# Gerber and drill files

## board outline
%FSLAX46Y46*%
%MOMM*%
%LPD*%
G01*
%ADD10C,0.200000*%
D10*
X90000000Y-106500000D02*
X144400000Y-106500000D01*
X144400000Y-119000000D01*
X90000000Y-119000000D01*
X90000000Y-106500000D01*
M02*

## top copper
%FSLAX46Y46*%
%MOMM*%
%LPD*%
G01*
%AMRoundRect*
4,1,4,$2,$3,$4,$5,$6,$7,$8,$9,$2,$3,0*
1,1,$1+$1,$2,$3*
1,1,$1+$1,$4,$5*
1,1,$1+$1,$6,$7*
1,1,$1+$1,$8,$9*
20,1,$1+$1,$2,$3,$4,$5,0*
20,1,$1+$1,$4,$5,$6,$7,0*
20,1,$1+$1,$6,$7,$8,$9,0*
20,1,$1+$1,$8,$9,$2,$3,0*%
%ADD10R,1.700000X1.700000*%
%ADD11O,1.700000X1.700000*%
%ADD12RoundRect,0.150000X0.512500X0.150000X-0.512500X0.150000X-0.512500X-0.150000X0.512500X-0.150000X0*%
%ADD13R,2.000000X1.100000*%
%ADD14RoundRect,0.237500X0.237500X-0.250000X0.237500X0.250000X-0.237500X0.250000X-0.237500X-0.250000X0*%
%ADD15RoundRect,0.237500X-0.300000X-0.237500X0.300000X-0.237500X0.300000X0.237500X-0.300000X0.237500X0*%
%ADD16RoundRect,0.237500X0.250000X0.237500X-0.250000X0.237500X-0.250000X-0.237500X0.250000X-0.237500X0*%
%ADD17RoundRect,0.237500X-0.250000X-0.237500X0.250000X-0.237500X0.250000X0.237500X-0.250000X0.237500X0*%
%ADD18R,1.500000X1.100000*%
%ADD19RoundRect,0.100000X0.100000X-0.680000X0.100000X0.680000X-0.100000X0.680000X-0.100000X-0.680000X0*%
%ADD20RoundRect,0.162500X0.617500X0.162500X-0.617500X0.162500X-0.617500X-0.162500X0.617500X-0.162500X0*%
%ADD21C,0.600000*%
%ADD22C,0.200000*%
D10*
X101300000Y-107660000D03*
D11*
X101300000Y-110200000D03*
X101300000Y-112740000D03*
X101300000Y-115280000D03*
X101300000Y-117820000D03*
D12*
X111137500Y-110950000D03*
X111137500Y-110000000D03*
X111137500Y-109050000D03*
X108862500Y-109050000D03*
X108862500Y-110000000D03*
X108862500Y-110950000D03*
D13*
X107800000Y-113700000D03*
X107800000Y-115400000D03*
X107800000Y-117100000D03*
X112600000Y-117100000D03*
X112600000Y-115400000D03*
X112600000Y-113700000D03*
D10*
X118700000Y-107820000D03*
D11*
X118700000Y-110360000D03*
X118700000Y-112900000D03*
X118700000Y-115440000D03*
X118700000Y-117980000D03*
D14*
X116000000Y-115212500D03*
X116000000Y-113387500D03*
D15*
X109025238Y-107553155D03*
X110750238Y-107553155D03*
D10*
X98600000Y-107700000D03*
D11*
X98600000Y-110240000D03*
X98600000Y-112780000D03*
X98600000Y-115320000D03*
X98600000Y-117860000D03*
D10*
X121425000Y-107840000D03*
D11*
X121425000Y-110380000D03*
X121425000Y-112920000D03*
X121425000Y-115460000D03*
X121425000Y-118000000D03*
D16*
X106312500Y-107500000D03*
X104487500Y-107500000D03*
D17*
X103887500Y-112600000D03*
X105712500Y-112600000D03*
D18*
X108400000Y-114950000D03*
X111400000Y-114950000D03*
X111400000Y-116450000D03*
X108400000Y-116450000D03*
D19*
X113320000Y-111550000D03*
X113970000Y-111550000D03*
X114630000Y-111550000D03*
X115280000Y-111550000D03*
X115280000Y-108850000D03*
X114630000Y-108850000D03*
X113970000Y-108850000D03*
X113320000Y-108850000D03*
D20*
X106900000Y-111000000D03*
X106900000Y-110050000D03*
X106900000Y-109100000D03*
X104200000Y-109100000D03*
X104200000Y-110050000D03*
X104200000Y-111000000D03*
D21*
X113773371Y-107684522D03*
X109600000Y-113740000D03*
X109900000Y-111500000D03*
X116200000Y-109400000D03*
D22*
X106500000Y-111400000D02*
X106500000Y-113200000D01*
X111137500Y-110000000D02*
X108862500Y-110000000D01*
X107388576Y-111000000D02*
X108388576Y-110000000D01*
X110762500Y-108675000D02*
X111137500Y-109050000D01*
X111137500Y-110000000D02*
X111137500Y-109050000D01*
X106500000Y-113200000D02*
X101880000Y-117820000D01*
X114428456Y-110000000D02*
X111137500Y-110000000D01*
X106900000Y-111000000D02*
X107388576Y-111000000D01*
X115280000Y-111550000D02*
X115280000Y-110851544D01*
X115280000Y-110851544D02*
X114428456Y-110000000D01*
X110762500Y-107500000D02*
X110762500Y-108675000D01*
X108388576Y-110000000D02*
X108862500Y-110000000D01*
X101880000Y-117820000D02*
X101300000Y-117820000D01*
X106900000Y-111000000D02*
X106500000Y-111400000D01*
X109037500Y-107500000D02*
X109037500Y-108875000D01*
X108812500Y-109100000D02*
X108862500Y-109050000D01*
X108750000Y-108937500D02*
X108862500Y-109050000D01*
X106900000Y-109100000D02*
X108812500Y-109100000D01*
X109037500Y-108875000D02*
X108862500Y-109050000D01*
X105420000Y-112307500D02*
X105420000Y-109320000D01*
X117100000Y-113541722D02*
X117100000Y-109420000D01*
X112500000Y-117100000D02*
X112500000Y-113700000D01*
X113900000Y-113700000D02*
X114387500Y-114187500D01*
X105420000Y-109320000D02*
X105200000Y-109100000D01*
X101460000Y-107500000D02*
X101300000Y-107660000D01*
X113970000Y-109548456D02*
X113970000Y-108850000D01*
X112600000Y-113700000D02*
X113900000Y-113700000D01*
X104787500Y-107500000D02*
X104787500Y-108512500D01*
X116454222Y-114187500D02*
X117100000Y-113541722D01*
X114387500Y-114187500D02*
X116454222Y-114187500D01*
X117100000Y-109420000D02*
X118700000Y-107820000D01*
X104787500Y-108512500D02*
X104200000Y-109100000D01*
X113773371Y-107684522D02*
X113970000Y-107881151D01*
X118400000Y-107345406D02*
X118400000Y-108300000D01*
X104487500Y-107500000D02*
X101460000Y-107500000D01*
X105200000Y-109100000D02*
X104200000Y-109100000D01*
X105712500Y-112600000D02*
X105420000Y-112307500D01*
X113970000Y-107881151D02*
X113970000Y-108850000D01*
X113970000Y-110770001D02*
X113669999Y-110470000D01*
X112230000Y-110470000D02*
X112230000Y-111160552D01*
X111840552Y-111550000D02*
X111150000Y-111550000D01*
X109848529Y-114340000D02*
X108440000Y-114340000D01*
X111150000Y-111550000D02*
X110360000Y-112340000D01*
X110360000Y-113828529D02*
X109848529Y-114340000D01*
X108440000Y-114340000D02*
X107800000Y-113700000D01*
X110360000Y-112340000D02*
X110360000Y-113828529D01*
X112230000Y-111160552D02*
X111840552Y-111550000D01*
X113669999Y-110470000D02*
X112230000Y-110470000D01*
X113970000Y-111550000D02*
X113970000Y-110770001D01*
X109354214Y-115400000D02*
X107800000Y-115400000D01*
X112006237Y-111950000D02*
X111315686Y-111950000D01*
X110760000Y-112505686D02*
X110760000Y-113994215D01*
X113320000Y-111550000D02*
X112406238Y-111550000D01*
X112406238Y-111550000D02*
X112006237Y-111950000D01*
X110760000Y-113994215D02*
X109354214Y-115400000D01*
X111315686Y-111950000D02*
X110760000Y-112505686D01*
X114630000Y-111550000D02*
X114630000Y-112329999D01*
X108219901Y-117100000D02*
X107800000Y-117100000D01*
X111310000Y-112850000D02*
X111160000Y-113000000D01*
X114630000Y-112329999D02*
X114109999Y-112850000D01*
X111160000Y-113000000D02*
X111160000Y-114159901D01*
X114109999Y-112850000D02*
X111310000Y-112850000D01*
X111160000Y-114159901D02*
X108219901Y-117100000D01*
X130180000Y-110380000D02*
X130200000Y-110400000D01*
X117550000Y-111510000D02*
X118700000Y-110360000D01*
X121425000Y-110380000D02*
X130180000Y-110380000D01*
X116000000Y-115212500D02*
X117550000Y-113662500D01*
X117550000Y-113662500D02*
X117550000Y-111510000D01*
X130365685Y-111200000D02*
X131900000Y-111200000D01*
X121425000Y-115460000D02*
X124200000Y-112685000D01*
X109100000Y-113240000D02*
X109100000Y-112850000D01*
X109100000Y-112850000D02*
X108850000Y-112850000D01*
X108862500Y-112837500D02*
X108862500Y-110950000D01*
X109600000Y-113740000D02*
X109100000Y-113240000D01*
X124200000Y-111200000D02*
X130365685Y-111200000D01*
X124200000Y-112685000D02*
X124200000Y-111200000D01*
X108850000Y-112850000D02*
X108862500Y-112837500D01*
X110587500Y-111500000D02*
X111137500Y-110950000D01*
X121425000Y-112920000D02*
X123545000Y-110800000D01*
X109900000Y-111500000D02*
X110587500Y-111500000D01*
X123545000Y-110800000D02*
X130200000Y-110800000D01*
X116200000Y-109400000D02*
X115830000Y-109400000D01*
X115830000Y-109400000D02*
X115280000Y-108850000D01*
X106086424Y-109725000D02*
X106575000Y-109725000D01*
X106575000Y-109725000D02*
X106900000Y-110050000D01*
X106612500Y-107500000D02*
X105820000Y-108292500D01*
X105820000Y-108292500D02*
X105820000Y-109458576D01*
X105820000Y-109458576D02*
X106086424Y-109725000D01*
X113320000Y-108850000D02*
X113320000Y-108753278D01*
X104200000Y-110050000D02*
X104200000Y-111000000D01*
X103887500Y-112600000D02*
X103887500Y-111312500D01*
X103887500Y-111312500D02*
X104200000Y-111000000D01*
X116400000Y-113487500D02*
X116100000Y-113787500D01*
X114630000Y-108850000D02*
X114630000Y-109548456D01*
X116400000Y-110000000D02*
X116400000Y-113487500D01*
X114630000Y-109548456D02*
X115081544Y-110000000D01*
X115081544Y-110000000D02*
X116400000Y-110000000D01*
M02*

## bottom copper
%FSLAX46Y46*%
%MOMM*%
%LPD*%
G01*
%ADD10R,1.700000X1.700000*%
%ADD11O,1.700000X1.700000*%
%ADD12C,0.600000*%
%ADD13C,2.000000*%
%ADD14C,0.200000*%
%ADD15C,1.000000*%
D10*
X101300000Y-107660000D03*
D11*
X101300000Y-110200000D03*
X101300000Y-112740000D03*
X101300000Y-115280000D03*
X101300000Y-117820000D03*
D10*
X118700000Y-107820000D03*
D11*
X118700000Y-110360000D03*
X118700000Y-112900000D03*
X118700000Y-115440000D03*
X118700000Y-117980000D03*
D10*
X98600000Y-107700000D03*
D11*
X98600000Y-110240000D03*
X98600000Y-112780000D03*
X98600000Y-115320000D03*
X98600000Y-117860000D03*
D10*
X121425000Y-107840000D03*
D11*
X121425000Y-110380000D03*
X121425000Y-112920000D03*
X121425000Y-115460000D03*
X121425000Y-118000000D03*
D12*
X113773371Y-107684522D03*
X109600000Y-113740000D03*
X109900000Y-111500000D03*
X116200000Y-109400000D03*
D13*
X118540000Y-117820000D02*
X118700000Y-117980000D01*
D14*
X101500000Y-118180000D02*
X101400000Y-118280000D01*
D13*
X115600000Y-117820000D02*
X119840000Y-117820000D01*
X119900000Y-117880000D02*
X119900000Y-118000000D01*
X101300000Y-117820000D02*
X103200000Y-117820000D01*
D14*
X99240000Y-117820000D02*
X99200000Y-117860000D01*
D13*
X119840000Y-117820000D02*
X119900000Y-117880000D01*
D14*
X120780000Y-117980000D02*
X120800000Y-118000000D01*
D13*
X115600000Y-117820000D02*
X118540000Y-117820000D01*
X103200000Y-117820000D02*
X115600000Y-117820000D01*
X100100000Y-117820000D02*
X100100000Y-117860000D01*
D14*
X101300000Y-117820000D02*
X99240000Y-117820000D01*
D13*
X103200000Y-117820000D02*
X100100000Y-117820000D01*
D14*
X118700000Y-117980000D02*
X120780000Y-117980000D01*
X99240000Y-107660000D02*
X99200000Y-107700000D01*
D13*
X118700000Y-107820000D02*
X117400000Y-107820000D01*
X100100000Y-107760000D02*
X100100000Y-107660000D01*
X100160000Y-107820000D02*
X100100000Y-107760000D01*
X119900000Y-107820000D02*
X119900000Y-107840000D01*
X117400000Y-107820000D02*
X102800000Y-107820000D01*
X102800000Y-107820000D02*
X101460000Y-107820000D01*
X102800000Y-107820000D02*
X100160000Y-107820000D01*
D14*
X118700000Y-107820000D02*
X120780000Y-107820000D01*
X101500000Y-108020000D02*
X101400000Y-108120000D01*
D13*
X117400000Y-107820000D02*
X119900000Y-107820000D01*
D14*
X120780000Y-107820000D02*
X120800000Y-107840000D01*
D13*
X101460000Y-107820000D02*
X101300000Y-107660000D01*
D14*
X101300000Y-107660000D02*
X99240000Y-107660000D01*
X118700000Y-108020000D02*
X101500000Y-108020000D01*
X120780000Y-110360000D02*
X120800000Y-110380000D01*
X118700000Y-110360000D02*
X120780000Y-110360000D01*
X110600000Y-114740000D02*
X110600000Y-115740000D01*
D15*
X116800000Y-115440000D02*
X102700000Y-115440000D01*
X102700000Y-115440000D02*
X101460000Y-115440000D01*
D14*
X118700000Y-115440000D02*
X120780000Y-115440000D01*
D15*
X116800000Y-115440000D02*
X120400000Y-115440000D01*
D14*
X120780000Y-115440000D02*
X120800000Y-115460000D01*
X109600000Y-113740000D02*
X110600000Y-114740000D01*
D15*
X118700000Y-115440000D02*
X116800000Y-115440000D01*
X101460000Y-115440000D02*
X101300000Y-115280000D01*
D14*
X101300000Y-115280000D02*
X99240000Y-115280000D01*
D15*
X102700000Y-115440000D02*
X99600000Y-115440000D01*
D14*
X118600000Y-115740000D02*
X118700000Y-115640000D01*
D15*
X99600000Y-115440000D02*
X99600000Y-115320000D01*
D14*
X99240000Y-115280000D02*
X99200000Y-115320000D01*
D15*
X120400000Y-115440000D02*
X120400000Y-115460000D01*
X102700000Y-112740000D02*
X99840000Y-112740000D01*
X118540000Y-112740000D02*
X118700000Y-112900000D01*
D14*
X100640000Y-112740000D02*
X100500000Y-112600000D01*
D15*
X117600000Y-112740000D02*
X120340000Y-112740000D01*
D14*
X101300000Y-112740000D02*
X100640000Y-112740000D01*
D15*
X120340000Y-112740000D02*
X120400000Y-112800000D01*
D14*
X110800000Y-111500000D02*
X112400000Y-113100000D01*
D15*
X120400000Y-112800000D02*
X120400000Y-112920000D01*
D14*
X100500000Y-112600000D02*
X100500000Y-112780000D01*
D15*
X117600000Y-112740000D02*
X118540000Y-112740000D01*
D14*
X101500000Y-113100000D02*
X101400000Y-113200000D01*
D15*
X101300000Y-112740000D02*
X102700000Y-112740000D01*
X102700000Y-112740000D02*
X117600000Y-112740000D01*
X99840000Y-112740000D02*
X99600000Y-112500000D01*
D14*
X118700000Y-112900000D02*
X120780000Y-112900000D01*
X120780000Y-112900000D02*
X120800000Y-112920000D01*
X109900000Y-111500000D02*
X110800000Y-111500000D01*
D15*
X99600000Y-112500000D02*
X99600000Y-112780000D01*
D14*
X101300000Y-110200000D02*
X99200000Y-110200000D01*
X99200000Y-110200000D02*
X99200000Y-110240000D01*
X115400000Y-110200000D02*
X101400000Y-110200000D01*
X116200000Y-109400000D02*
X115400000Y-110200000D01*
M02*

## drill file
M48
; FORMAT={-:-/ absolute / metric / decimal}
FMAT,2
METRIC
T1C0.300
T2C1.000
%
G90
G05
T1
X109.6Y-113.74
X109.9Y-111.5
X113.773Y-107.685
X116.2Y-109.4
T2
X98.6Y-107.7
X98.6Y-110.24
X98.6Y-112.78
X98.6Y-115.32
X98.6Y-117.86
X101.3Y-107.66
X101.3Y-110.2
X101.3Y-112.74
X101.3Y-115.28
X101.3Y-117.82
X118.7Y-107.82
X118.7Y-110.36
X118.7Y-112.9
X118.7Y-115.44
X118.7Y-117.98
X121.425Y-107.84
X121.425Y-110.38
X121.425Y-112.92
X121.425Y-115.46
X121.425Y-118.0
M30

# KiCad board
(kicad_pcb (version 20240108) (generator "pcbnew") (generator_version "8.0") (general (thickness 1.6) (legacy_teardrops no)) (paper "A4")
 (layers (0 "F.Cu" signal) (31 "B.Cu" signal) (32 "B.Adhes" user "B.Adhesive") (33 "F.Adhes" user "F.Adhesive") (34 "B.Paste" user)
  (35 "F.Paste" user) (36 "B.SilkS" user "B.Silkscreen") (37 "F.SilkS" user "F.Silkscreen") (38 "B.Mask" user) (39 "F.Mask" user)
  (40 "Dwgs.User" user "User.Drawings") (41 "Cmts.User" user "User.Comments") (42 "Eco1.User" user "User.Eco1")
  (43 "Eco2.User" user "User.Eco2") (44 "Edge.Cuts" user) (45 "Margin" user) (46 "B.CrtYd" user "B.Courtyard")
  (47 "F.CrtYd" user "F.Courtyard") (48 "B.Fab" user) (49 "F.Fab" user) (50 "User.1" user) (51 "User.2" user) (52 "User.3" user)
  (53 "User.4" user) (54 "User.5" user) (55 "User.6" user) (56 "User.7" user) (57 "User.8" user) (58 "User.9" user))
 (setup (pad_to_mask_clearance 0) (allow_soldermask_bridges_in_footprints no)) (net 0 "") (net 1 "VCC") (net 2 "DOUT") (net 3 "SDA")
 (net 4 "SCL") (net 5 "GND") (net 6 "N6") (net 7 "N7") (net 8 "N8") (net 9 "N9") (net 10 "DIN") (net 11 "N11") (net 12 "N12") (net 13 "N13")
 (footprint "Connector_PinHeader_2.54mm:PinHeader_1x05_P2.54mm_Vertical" (layer "F.Cu") (at 101.3 107.66)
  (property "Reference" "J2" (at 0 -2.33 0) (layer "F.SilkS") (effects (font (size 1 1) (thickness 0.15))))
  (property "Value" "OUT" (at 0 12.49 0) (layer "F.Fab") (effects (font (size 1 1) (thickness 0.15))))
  (pad "1" thru_hole rect (at 0 0) (size 1.7 1.7) (drill 1) (layers "*.Cu" "*.Mask") (remove_unused_layers no) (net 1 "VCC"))
  (pad "2" thru_hole oval (at 0 2.54) (size 1.7 1.7) (drill 1) (layers "*.Cu" "*.Mask") (remove_unused_layers no) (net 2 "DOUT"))
  (pad "3" thru_hole oval (at 0 5.08) (size 1.7 1.7) (drill 1) (layers "*.Cu" "*.Mask") (remove_unused_layers no) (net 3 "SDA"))
  (pad "4" thru_hole oval (at 0 7.62) (size 1.7 1.7) (drill 1) (layers "*.Cu" "*.Mask") (remove_unused_layers no) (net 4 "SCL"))
  (pad "5" thru_hole oval (at 0 10.16) (size 1.7 1.7) (drill 1) (layers "*.Cu" "*.Mask") (remove_unused_layers no) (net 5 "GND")))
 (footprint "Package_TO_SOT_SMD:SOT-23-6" (layer "F.Cu") (at 110 110 180)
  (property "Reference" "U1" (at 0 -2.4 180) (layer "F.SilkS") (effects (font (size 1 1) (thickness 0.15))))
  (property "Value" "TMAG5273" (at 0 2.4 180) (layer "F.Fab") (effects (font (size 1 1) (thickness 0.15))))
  (pad "1" smd roundrect (at -1.1375 -0.95 180) (size 1.325 0.6) (layers "F.Cu" "F.Paste" "F.Mask") (roundrect_rratio 0.25) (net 3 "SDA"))
  (pad "2" smd roundrect (at -1.1375 0 180) (size 1.325 0.6) (layers "F.Cu" "F.Paste" "F.Mask") (roundrect_rratio 0.25) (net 5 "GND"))
  (pad "3" smd roundrect (at -1.1375 0.95 180) (size 1.325 0.6) (layers "F.Cu" "F.Paste" "F.Mask") (roundrect_rratio 0.25) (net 5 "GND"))
  (pad "4" smd roundrect (at 1.1375 0.95 180) (size 1.325 0.6) (layers "F.Cu" "F.Paste" "F.Mask") (roundrect_rratio 0.25) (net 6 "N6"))
  (pad "5" smd roundrect (at 1.1375 0 180) (size 1.325 0.6) (layers "F.Cu" "F.Paste" "F.Mask") (roundrect_rratio 0.25) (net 5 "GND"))
  (pad "6" smd roundrect (at 1.1375 -0.95 180) (size 1.325 0.6) (layers "F.Cu" "F.Paste" "F.Mask") (roundrect_rratio 0.25) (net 4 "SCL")))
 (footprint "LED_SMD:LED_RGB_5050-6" (layer "F.Cu") (at 110.2 115.4)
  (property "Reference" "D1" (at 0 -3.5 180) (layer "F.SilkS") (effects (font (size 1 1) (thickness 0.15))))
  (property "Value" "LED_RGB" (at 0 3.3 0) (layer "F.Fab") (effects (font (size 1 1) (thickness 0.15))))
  (pad "1" smd rect (at -2.4 -1.7 90) (size 1.1 2) (layers "F.Cu" "F.Paste" "F.Mask") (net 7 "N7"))
  (pad "2" smd rect (at -2.4 0 90) (size 1.1 2) (layers "F.Cu" "F.Paste" "F.Mask") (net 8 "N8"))
  (pad "3" smd rect (at -2.4 1.7 90) (size 1.1 2) (layers "F.Cu" "F.Paste" "F.Mask") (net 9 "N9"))
  (pad "4" smd rect (at 2.4 1.7 90) (size 1.1 2) (layers "F.Cu" "F.Paste" "F.Mask") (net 1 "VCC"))
  (pad "5" smd rect (at 2.4 0 90) (size 1.1 2) (layers "F.Cu" "F.Paste" "F.Mask") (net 1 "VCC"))
  (pad "6" smd rect (at 2.4 -1.7 90) (size 1.1 2) (layers "F.Cu" "F.Paste" "F.Mask") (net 1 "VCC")))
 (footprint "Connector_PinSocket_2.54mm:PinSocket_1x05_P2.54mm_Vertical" (layer "F.Cu") (at 118.7 107.82)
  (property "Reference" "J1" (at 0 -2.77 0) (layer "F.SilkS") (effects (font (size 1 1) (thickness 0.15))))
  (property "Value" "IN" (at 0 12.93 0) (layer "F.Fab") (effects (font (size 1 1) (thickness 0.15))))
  (pad "1" thru_hole rect (at 0 0) (size 1.7 1.7) (drill 1) (layers "*.Cu" "*.Mask") (remove_unused_layers no) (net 1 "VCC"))
  (pad "2" thru_hole oval (at 0 2.54) (size 1.7 1.7) (drill 1) (layers "*.Cu" "*.Mask") (remove_unused_layers no) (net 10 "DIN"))
  (pad "3" thru_hole oval (at 0 5.08) (size 1.7 1.7) (drill 1) (layers "*.Cu" "*.Mask") (remove_unused_layers no) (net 3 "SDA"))
  (pad "4" thru_hole oval (at 0 7.62) (size 1.7 1.7) (drill 1) (layers "*.Cu" "*.Mask") (remove_unused_layers no) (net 4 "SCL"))
  (pad "5" thru_hole oval (at 0 10.16) (size 1.7 1.7) (drill 1) (layers "*.Cu" "*.Mask") (remove_unused_layers no) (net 5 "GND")))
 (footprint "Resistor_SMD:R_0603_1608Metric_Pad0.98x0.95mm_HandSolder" (layer "F.Cu") (at 116 114.3 90)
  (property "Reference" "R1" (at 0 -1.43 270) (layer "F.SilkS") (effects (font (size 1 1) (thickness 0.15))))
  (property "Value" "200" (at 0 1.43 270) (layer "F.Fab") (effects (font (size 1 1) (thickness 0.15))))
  (pad "1" smd roundrect (at -0.9125 0 90) (size 0.975 0.95) (layers "F.Cu" "F.Paste" "F.Mask") (roundrect_rratio 0.25) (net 10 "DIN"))
  (pad "2" smd roundrect (at 0.9125 0 90) (size 0.975 0.95) (layers "F.Cu" "F.Paste" "F.Mask") (roundrect_rratio 0.25) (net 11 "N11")))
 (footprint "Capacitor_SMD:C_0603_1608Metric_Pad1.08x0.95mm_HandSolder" (layer "F.Cu") (at 109.887738 107.553155)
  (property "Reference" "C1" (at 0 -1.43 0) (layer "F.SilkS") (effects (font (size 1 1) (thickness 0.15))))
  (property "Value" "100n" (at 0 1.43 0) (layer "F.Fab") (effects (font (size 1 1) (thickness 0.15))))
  (pad "1" smd roundrect (at -0.8625 0) (size 1.075 0.95) (layers "F.Cu" "F.Paste" "F.Mask") (roundrect_rratio 0.25) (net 6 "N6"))
  (pad "2" smd roundrect (at 0.8625 0) (size 1.075 0.95) (layers "F.Cu" "F.Paste" "F.Mask") (roundrect_rratio 0.25) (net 5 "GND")))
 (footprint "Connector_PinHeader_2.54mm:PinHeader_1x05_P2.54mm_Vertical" (layer "F.Cu") (at 98.6 107.7)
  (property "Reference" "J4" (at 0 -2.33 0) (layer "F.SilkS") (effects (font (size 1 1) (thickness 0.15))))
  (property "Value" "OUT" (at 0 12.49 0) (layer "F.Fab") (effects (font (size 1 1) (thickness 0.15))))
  (pad "1" thru_hole rect (at 0 0) (size 1.7 1.7) (drill 1) (layers "*.Cu" "*.Mask") (remove_unused_layers no) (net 1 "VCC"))
  (pad "2" thru_hole oval (at 0 2.54) (size 1.7 1.7) (drill 1) (layers "*.Cu" "*.Mask") (remove_unused_layers no) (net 2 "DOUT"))
  (pad "3" thru_hole oval (at 0 5.08) (size 1.7 1.7) (drill 1) (layers "*.Cu" "*.Mask") (remove_unused_layers no) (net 3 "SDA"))
  (pad "4" thru_hole oval (at 0 7.62) (size 1.7 1.7) (drill 1) (layers "*.Cu" "*.Mask") (remove_unused_layers no) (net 4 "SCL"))
  (pad "5" thru_hole oval (at 0 10.16) (size 1.7 1.7) (drill 1) (layers "*.Cu" "*.Mask") (remove_unused_layers no) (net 5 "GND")))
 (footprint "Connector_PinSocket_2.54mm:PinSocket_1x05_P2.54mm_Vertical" (layer "F.Cu") (at 121.425 107.84)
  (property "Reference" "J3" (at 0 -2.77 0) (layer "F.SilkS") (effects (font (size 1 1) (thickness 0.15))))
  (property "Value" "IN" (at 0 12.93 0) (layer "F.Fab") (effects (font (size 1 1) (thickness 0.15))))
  (pad "1" thru_hole rect (at 0 0) (size 1.7 1.7) (drill 1) (layers "*.Cu" "*.Mask") (remove_unused_layers no) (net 1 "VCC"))
  (pad "2" thru_hole oval (at 0 2.54) (size 1.7 1.7) (drill 1) (layers "*.Cu" "*.Mask") (remove_unused_layers no) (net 10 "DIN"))
  (pad "3" thru_hole oval (at 0 5.08) (size 1.7 1.7) (drill 1) (layers "*.Cu" "*.Mask") (remove_unused_layers no) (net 3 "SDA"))
  (pad "4" thru_hole oval (at 0 7.62) (size 1.7 1.7) (drill 1) (layers "*.Cu" "*.Mask") (remove_unused_layers no) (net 4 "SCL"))
  (pad "5" thru_hole oval (at 0 10.16) (size 1.7 1.7) (drill 1) (layers "*.Cu" "*.Mask") (remove_unused_layers no) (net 5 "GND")))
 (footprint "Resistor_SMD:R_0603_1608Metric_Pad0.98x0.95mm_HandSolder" (layer "F.Cu") (at 105.4 107.5 180)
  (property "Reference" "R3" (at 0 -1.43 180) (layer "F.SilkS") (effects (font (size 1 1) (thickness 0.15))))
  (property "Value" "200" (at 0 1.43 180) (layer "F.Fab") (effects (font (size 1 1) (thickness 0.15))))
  (pad "1" smd roundrect (at -0.9125 0 180) (size 0.975 0.95) (layers "F.Cu" "F.Paste" "F.Mask") (roundrect_rratio 0.25) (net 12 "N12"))
  (pad "2" smd roundrect (at 0.9125 0 180) (size 0.975 0.95) (layers "F.Cu" "F.Paste" "F.Mask") (roundrect_rratio 0.25) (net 1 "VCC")))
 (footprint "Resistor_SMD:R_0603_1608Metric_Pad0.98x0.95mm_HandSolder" (layer "F.Cu") (at 104.8 112.6)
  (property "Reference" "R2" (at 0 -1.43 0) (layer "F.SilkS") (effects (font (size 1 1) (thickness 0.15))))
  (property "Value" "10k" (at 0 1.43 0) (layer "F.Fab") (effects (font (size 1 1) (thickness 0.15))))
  (pad "1" smd roundrect (at -0.9125 0) (size 0.975 0.95) (layers "F.Cu" "F.Paste" "F.Mask") (roundrect_rratio 0.25) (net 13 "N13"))
  (pad "2" smd roundrect (at 0.9125 0) (size 0.975 0.95) (layers "F.Cu" "F.Paste" "F.Mask") (roundrect_rratio 0.25) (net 1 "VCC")))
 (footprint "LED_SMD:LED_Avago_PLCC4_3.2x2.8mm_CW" (layer "F.Cu") (at 109.9 115.7)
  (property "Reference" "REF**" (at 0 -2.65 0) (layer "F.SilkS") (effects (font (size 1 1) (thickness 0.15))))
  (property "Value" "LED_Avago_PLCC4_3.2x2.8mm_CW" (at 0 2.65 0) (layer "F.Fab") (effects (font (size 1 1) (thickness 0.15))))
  (pad "1" smd rect (at -1.5 -0.75) (size 1.5 1.1) (layers "F.Cu" "F.Paste" "F.Mask"))
  (pad "2" smd rect (at 1.5 -0.75) (size 1.5 1.1) (layers "F.Cu" "F.Paste" "F.Mask"))
  (pad "3" smd rect (at 1.5 0.75) (size 1.5 1.1) (layers "F.Cu" "F.Paste" "F.Mask"))
  (pad "4" smd rect (at -1.5 0.75) (size 1.5 1.1) (layers "F.Cu" "F.Paste" "F.Mask")))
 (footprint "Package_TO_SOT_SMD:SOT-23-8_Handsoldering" (layer "F.Cu") (at 114.3 110.2 90)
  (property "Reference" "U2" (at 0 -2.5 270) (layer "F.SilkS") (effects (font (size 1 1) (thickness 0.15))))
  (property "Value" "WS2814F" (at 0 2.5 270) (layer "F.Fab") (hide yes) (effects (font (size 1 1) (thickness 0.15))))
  (pad "1" smd roundrect (at -1.35 -0.98 90) (size 1.56 0.4) (layers "F.Cu" "F.Paste" "F.Mask") (roundrect_rratio 0.25) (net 8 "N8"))
  (pad "2" smd roundrect (at -1.35 -0.33 90) (size 1.56 0.4) (layers "F.Cu" "F.Paste" "F.Mask") (roundrect_rratio 0.25) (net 7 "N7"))
  (pad "3" smd roundrect (at -1.35 0.33 90) (size 1.56 0.4) (layers "F.Cu" "F.Paste" "F.Mask") (roundrect_rratio 0.25) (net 9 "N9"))
  (pad "4" smd roundrect (at -1.35 0.98 90) (size 1.56 0.4) (layers "F.Cu" "F.Paste" "F.Mask") (roundrect_rratio 0.25) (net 5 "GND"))
  (pad "5" smd roundrect (at 1.35 0.98 90) (size 1.56 0.4) (layers "F.Cu" "F.Paste" "F.Mask") (roundrect_rratio 0.25) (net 2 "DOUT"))
  (pad "6" smd roundrect (at 1.35 0.33 90) (size 1.56 0.4) (layers "F.Cu" "F.Paste" "F.Mask") (roundrect_rratio 0.25) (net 11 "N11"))
  (pad "7" smd roundrect (at 1.35 -0.33 90) (size 1.56 0.4) (layers "F.Cu" "F.Paste" "F.Mask") (roundrect_rratio 0.25) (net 1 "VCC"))
  (pad "8" smd roundrect (at 1.35 -0.98 90) (size 1.56 0.4) (layers "F.Cu" "F.Paste" "F.Mask") (roundrect_rratio 0.25) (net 12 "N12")))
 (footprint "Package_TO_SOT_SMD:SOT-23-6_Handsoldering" (layer "F.Cu") (at 105.55 110.05 180)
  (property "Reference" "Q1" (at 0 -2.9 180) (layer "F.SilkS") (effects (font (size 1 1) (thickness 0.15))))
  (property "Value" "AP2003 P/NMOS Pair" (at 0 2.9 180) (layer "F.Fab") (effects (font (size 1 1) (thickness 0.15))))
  (pad "1" smd roundrect (at -1.35 -0.95 180) (size 1.56 0.65) (layers "F.Cu" "F.Paste" "F.Mask") (roundrect_rratio 0.25) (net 5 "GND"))
  (pad "2" smd roundrect (at -1.35 0 180) (size 1.56 0.65) (layers "F.Cu" "F.Paste" "F.Mask") (roundrect_rratio 0.25) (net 12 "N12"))
  (pad "3" smd roundrect (at -1.35 0.95 180) (size 1.56 0.65) (layers "F.Cu" "F.Paste" "F.Mask") (roundrect_rratio 0.25) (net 6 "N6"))
  (pad "4" smd roundrect (at 1.35 0.95 180) (size 1.56 0.65) (layers "F.Cu" "F.Paste" "F.Mask") (roundrect_rratio 0.25) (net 1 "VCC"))
  (pad "5" smd roundrect (at 1.35 0 180) (size 1.56 0.65) (layers "F.Cu" "F.Paste" "F.Mask") (roundrect_rratio 0.25) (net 13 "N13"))
  (pad "6" smd roundrect (at 1.35 -0.95 180) (size 1.56 0.65) (layers "F.Cu" "F.Paste" "F.Mask") (roundrect_rratio 0.25) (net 13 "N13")))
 (gr_rect (start 90 106.5) (end 144.4 119) (stroke (width 0.2) (type default)) (fill none) (layer "Edge.Cuts"))
 (segment (start 106.5 111.4) (end 106.5 113.2) (width 0.2) (layer "F.Cu") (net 5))
 (segment (start 111.1375 110) (end 108.8625 110) (width 0.2) (layer "F.Cu") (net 5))
 (segment (start 107.388576 111) (end 108.388576 110) (width 0.2) (layer "F.Cu") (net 5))
 (segment (start 110.7625 108.675) (end 111.1375 109.05) (width 0.2) (layer "F.Cu") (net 5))
 (segment (start 111.1375 110) (end 111.1375 109.05) (width 0.2) (layer "F.Cu") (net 5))
 (segment (start 106.5 113.2) (end 101.88 117.82) (width 0.2) (layer "F.Cu") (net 5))
 (segment (start 114.428456 110) (end 111.1375 110) (width 0.2) (layer "F.Cu") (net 5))
 (segment (start 106.9 111) (end 107.388576 111) (width 0.2) (layer "F.Cu") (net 5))
 (segment (start 115.28 111.55) (end 115.28 110.851544) (width 0.2) (layer "F.Cu") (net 5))
 (segment (start 115.28 110.851544) (end 114.428456 110) (width 0.2) (layer "F.Cu") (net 5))
 (segment (start 110.7625 107.5) (end 110.7625 108.675) (width 0.2) (layer "F.Cu") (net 5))
 (segment (start 108.388576 110) (end 108.8625 110) (width 0.2) (layer "F.Cu") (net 5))
 (segment (start 101.88 117.82) (end 101.3 117.82) (width 0.2) (layer "F.Cu") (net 5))
 (segment (start 106.9 111) (end 106.5 111.4) (width 0.2) (layer "F.Cu") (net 5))
 (segment (start 118.54 117.82) (end 118.7 117.98) (width 2) (layer "B.Cu") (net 5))
 (segment (start 101.5 118.18) (end 101.4 118.28) (width 0.2) (layer "B.Cu") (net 5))
 (segment (start 115.6 117.82) (end 119.84 117.82) (width 2) (layer "B.Cu") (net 5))
 (segment (start 119.9 117.88) (end 119.9 118) (width 2) (layer "B.Cu") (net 5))
 (segment (start 101.3 117.82) (end 103.2 117.82) (width 2) (layer "B.Cu") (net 5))
 (segment (start 99.24 117.82) (end 99.2 117.86) (width 0.2) (layer "B.Cu") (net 5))
 (segment (start 119.84 117.82) (end 119.9 117.88) (width 2) (layer "B.Cu") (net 5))
 (segment (start 120.78 117.98) (end 120.8 118) (width 0.2) (layer "B.Cu") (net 5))
 (segment (start 115.6 117.82) (end 118.54 117.82) (width 2) (layer "B.Cu") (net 5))
 (segment (start 103.2 117.82) (end 115.6 117.82) (width 2) (layer "B.Cu") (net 5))
 (segment (start 100.1 117.82) (end 100.1 117.86) (width 2) (layer "B.Cu") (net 5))
 (segment (start 101.3 117.82) (end 99.24 117.82) (width 0.2) (layer "B.Cu") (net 5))
 (segment (start 103.2 117.82) (end 100.1 117.82) (width 2) (layer "B.Cu") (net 5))
 (segment (start 118.7 117.98) (end 120.78 117.98) (width 0.2) (layer "B.Cu") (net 5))
 (segment (start 109.0375 107.5) (end 109.0375 108.875) (width 0.2) (layer "F.Cu") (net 6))
 (segment (start 108.8125 109.1) (end 108.8625 109.05) (width 0.2) (layer "F.Cu") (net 6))
 (segment (start 108.75 108.9375) (end 108.8625 109.05) (width 0.2) (layer "F.Cu") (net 6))
 (segment (start 106.9 109.1) (end 108.8125 109.1) (width 0.2) (layer "F.Cu") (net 6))
 (segment (start 109.0375 108.875) (end 108.8625 109.05) (width 0.2) (layer "F.Cu") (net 6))
 (segment (start 105.42 112.3075) (end 105.42 109.32) (width 0.2) (layer "F.Cu") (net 1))
 (segment (start 117.1 113.541722) (end 117.1 109.42) (width 0.2) (layer "F.Cu") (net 1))
 (segment (start 112.5 117.1) (end 112.5 113.7) (width 0.2) (layer "F.Cu") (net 1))
 (segment (start 113.9 113.7) (end 114.3875 114.1875) (width 0.2) (layer "F.Cu") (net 1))
 (segment (start 105.42 109.32) (end 105.2 109.1) (width 0.2) (layer "F.Cu") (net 1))
 (segment (start 101.46 107.5) (end 101.3 107.66) (width 0.2) (layer "F.Cu") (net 1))
 (segment (start 113.97 109.548456) (end 113.97 108.85) (width 0.2) (layer "F.Cu") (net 1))
 (segment (start 112.6 113.7) (end 113.9 113.7) (width 0.2) (layer "F.Cu") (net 1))
 (segment (start 104.7875 107.5) (end 104.7875 108.5125) (width 0.2) (layer "F.Cu") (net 1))
 (segment (start 116.454222 114.1875) (end 117.1 113.541722) (width 0.2) (layer "F.Cu") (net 1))
 (segment (start 114.3875 114.1875) (end 116.454222 114.1875) (width 0.2) (layer "F.Cu") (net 1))
 (segment (start 117.1 109.42) (end 118.7 107.82) (width 0.2) (layer "F.Cu") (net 1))
 (segment (start 104.7875 108.5125) (end 104.2 109.1) (width 0.2) (layer "F.Cu") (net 1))
 (segment (start 113.773371 107.684522) (end 113.97 107.881151) (width 0.2) (layer "F.Cu") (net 1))
 (segment (start 118.4 107.345406) (end 118.4 108.3) (width 0.2) (layer "F.Cu") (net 1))
 (segment (start 104.4875 107.5) (end 101.46 107.5) (width 0.2) (layer "F.Cu") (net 1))
 (segment (start 105.2 109.1) (end 104.2 109.1) (width 0.2) (layer "F.Cu") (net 1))
 (segment (start 105.7125 112.6) (end 105.42 112.3075) (width 0.2) (layer "F.Cu") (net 1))
 (segment (start 113.97 107.881151) (end 113.97 108.85) (width 0.2) (layer "F.Cu") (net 1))
 (via (at 113.773371 107.684522) (size 0.6) (drill 0.3) (layers "F.Cu" "B.Cu") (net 1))
 (segment (start 99.24 107.66) (end 99.2 107.7) (width 0.2) (layer "B.Cu") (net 1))
 (segment (start 118.7 107.82) (end 117.4 107.82) (width 2) (layer "B.Cu") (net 1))
 (segment (start 100.1 107.76) (end 100.1 107.66) (width 2) (layer "B.Cu") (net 1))
 (segment (start 100.16 107.82) (end 100.1 107.76) (width 2) (layer "B.Cu") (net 1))
 (segment (start 119.9 107.82) (end 119.9 107.84) (width 2) (layer "B.Cu") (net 1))
 (segment (start 117.4 107.82) (end 102.8 107.82) (width 2) (layer "B.Cu") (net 1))
 (segment (start 102.8 107.82) (end 101.46 107.82) (width 2) (layer "B.Cu") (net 1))
 (segment (start 102.8 107.82) (end 100.16 107.82) (width 2) (layer "B.Cu") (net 1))
 (segment (start 118.7 107.82) (end 120.78 107.82) (width 0.2) (layer "B.Cu") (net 1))
 (segment (start 101.5 108.02) (end 101.4 108.12) (width 0.2) (layer "B.Cu") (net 1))
 (segment (start 117.4 107.82) (end 119.9 107.82) (width 2) (layer "B.Cu") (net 1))
 (segment (start 120.78 107.82) (end 120.8 107.84) (width 0.2) (layer "B.Cu") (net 1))
 (segment (start 101.46 107.82) (end 101.3 107.66) (width 2) (layer "B.Cu") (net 1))
 (segment (start 101.3 107.66) (end 99.24 107.66) (width 0.2) (layer "B.Cu") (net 1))
 (segment (start 118.7 108.02) (end 101.5 108.02) (width 0.2) (layer "B.Cu") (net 1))
 (segment (start 113.97 110.770001) (end 113.669999 110.47) (width 0.2) (layer "F.Cu") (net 7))
 (segment (start 112.23 110.47) (end 112.23 111.160552) (width 0.2) (layer "F.Cu") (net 7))
 (segment (start 111.840552 111.55) (end 111.15 111.55) (width 0.2) (layer "F.Cu") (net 7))
 (segment (start 109.848529 114.34) (end 108.44 114.34) (width 0.2) (layer "F.Cu") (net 7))
 (segment (start 111.15 111.55) (end 110.36 112.34) (width 0.2) (layer "F.Cu") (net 7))
 (segment (start 110.36 113.828529) (end 109.848529 114.34) (width 0.2) (layer "F.Cu") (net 7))
 (segment (start 108.44 114.34) (end 107.8 113.7) (width 0.2) (layer "F.Cu") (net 7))
 (segment (start 110.36 112.34) (end 110.36 113.828529) (width 0.2) (layer "F.Cu") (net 7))
 (segment (start 112.23 111.160552) (end 111.840552 111.55) (width 0.2) (layer "F.Cu") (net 7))
 (segment (start 113.669999 110.47) (end 112.23 110.47) (width 0.2) (layer "F.Cu") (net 7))
 (segment (start 113.97 111.55) (end 113.97 110.770001) (width 0.2) (layer "F.Cu") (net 7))
 (segment (start 109.354214 115.4) (end 107.8 115.4) (width 0.2) (layer "F.Cu") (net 8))
 (segment (start 112.006237 111.95) (end 111.315686 111.95) (width 0.2) (layer "F.Cu") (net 8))
 (segment (start 110.76 112.505686) (end 110.76 113.994215) (width 0.2) (layer "F.Cu") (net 8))
 (segment (start 113.32 111.55) (end 112.406238 111.55) (width 0.2) (layer "F.Cu") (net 8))
 (segment (start 112.406238 111.55) (end 112.006237 111.95) (width 0.2) (layer "F.Cu") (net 8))
 (segment (start 110.76 113.994215) (end 109.354214 115.4) (width 0.2) (layer "F.Cu") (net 8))
 (segment (start 111.315686 111.95) (end 110.76 112.505686) (width 0.2) (layer "F.Cu") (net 8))
 (segment (start 114.63 111.55) (end 114.63 112.329999) (width 0.2) (layer "F.Cu") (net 9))
 (segment (start 108.219901 117.1) (end 107.8 117.1) (width 0.2) (layer "F.Cu") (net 9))
 (segment (start 111.31 112.85) (end 111.16 113) (width 0.2) (layer "F.Cu") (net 9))
 (segment (start 114.63 112.329999) (end 114.109999 112.85) (width 0.2) (layer "F.Cu") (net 9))
 (segment (start 111.16 113) (end 111.16 114.159901) (width 0.2) (layer "F.Cu") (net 9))
 (segment (start 114.109999 112.85) (end 111.31 112.85) (width 0.2) (layer "F.Cu") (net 9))
 (segment (start 111.16 114.159901) (end 108.219901 117.1) (width 0.2) (layer "F.Cu") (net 9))
 (segment (start 130.18 110.38) (end 130.2 110.4) (width 0.2) (layer "F.Cu") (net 10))
 (segment (start 117.55 111.51) (end 118.7 110.36) (width 0.2) (layer "F.Cu") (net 10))
 (segment (start 121.425 110.38) (end 130.18 110.38) (width 0.2) (layer "F.Cu") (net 10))
 (segment (start 116 115.2125) (end 117.55 113.6625) (width 0.2) (layer "F.Cu") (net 10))
 (segment (start 117.55 113.6625) (end 117.55 111.51) (width 0.2) (layer "F.Cu") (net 10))
 (segment (start 120.78 110.36) (end 120.8 110.38) (width 0.2) (layer "B.Cu") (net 10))
 (segment (start 118.7 110.36) (end 120.78 110.36) (width 0.2) (layer "B.Cu") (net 10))
 (segment (start 130.365685 111.2) (end 131.9 111.2) (width 0.2) (layer "F.Cu") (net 4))
 (segment (start 121.425 115.46) (end 124.2 112.685) (width 0.2) (layer "F.Cu") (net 4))
 (segment (start 109.1 113.24) (end 109.1 112.85) (width 0.2) (layer "F.Cu") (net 4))
 (segment (start 109.1 112.85) (end 108.85 112.85) (width 0.2) (layer "F.Cu") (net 4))
 (segment (start 108.8625 112.8375) (end 108.8625 110.95) (width 0.2) (layer "F.Cu") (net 4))
 (segment (start 109.6 113.74) (end 109.1 113.24) (width 0.2) (layer "F.Cu") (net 4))
 (segment (start 124.2 111.2) (end 130.365685 111.2) (width 0.2) (layer "F.Cu") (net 4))
 (segment (start 124.2 112.685) (end 124.2 111.2) (width 0.2) (layer "F.Cu") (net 4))
 (segment (start 108.85 112.85) (end 108.8625 112.8375) (width 0.2) (layer "F.Cu") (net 4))
 (via (at 109.6 113.74) (size 0.6) (drill 0.3) (layers "F.Cu" "B.Cu") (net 4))
 (segment (start 110.6 114.74) (end 110.6 115.74) (width 0.2) (layer "B.Cu") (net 4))
 (segment (start 116.8 115.44) (end 102.7 115.44) (width 1) (layer "B.Cu") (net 4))
 (segment (start 102.7 115.44) (end 101.46 115.44) (width 1) (layer "B.Cu") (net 4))
 (segment (start 118.7 115.44) (end 120.78 115.44) (width 0.2) (layer "B.Cu") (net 4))
 (segment (start 116.8 115.44) (end 120.4 115.44) (width 1) (layer "B.Cu") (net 4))
 (segment (start 120.78 115.44) (end 120.8 115.46) (width 0.2) (layer "B.Cu") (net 4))
 (segment (start 109.6 113.74) (end 110.6 114.74) (width 0.2) (layer "B.Cu") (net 4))
 (segment (start 118.7 115.44) (end 116.8 115.44) (width 1) (layer "B.Cu") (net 4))
 (segment (start 101.46 115.44) (end 101.3 115.28) (width 1) (layer "B.Cu") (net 4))
 (segment (start 101.3 115.28) (end 99.24 115.28) (width 0.2) (layer "B.Cu") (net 4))
 (segment (start 102.7 115.44) (end 99.6 115.44) (width 1) (layer "B.Cu") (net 4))
 (segment (start 118.6 115.74) (end 118.7 115.64) (width 0.2) (layer "B.Cu") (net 4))
 (segment (start 99.6 115.44) (end 99.6 115.32) (width 1) (layer "B.Cu") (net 4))
 (segment (start 99.24 115.28) (end 99.2 115.32) (width 0.2) (layer "B.Cu") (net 4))
 (segment (start 120.4 115.44) (end 120.4 115.46) (width 1) (layer "B.Cu") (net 4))
 (segment (start 110.5875 111.5) (end 111.1375 110.95) (width 0.2) (layer "F.Cu") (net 3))
 (segment (start 121.425 112.92) (end 123.545 110.8) (width 0.2) (layer "F.Cu") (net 3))
 (segment (start 109.9 111.5) (end 110.5875 111.5) (width 0.2) (layer "F.Cu") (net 3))
 (segment (start 123.545 110.8) (end 130.2 110.8) (width 0.2) (layer "F.Cu") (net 3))
 (via (at 109.9 111.5) (size 0.6) (drill 0.3) (layers "F.Cu" "B.Cu") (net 3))
 (segment (start 102.7 112.74) (end 99.84 112.74) (width 1) (layer "B.Cu") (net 3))
 (segment (start 118.54 112.74) (end 118.7 112.9) (width 1) (layer "B.Cu") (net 3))
 (segment (start 100.64 112.74) (end 100.5 112.6) (width 0.2) (layer "B.Cu") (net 3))
 (segment (start 117.6 112.74) (end 120.34 112.74) (width 1) (layer "B.Cu") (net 3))
 (segment (start 101.3 112.74) (end 100.64 112.74) (width 0.2) (layer "B.Cu") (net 3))
 (segment (start 120.34 112.74) (end 120.4 112.8) (width 1) (layer "B.Cu") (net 3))
 (segment (start 110.8 111.5) (end 112.4 113.1) (width 0.2) (layer "B.Cu") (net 3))
 (segment (start 120.4 112.8) (end 120.4 112.92) (width 1) (layer "B.Cu") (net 3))
 (segment (start 100.5 112.6) (end 100.5 112.78) (width 0.2) (layer "B.Cu") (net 3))
 (segment (start 117.6 112.74) (end 118.54 112.74) (width 1) (layer "B.Cu") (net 3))
 (segment (start 101.5 113.1) (end 101.4 113.2) (width 0.2) (layer "B.Cu") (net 3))
 (segment (start 101.3 112.74) (end 102.7 112.74) (width 1) (layer "B.Cu") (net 3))
 (segment (start 102.7 112.74) (end 117.6 112.74) (width 1) (layer "B.Cu") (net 3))
 (segment (start 99.84 112.74) (end 99.6 112.5) (width 1) (layer "B.Cu") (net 3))
 (segment (start 118.7 112.9) (end 120.78 112.9) (width 0.2) (layer "B.Cu") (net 3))
 (segment (start 120.78 112.9) (end 120.8 112.92) (width 0.2) (layer "B.Cu") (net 3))
 (segment (start 109.9 111.5) (end 110.8 111.5) (width 0.2) (layer "B.Cu") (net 3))
 (segment (start 99.6 112.5) (end 99.6 112.78) (width 1) (layer "B.Cu") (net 3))
 (segment (start 116.2 109.4) (end 115.83 109.4) (width 0.2) (layer "F.Cu") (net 2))
 (segment (start 115.83 109.4) (end 115.28 108.85) (width 0.2) (layer "F.Cu") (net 2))
 (via (at 116.2 109.4) (size 0.6) (drill 0.3) (layers "F.Cu" "B.Cu") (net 2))
 (segment (start 101.3 110.2) (end 99.2 110.2) (width 0.2) (layer "B.Cu") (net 2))
 (segment (start 99.2 110.2) (end 99.2 110.24) (width 0.2) (layer "B.Cu") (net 2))
 (segment (start 115.4 110.2) (end 101.4 110.2) (width 0.2) (layer "B.Cu") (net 2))
 (segment (start 116.2 109.4) (end 115.4 110.2) (width 0.2) (layer "B.Cu") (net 2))
 (segment (start 106.086424 109.725) (end 106.575 109.725) (width 0.2) (layer "F.Cu") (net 12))
 (segment (start 106.575 109.725) (end 106.9 110.05) (width 0.2) (layer "F.Cu") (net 12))
 (segment (start 106.6125 107.5) (end 105.82 108.2925) (width 0.2) (layer "F.Cu") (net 12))
 (segment (start 105.82 108.2925) (end 105.82 109.458576) (width 0.2) (layer "F.Cu") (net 12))
 (segment (start 105.82 109.458576) (end 106.086424 109.725) (width 0.2) (layer "F.Cu") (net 12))
 (segment (start 113.32 108.85) (end 113.32 108.753278) (width 0.2) (layer "F.Cu") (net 12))
 (segment (start 104.2 110.05) (end 104.2 111) (width 0.2) (layer "F.Cu") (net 13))
 (segment (start 103.8875 112.6) (end 103.8875 111.3125) (width 0.2) (layer "F.Cu") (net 13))
 (segment (start 103.8875 111.3125) (end 104.2 111) (width 0.2) (layer "F.Cu") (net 13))
 (segment (start 116.4 113.4875) (end 116.1 113.7875) (width 0.2) (layer "F.Cu") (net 11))
 (segment (start 114.63 108.85) (end 114.63 109.548456) (width 0.2) (layer "F.Cu") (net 11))
 (segment (start 116.4 110) (end 116.4 113.4875) (width 0.2) (layer "F.Cu") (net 11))
 (segment (start 114.63 109.548456) (end 115.081544 110) (width 0.2) (layer "F.Cu") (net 11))
 (segment (start 115.081544 110) (end 116.4 110) (width 0.2) (layer "F.Cu") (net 11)))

